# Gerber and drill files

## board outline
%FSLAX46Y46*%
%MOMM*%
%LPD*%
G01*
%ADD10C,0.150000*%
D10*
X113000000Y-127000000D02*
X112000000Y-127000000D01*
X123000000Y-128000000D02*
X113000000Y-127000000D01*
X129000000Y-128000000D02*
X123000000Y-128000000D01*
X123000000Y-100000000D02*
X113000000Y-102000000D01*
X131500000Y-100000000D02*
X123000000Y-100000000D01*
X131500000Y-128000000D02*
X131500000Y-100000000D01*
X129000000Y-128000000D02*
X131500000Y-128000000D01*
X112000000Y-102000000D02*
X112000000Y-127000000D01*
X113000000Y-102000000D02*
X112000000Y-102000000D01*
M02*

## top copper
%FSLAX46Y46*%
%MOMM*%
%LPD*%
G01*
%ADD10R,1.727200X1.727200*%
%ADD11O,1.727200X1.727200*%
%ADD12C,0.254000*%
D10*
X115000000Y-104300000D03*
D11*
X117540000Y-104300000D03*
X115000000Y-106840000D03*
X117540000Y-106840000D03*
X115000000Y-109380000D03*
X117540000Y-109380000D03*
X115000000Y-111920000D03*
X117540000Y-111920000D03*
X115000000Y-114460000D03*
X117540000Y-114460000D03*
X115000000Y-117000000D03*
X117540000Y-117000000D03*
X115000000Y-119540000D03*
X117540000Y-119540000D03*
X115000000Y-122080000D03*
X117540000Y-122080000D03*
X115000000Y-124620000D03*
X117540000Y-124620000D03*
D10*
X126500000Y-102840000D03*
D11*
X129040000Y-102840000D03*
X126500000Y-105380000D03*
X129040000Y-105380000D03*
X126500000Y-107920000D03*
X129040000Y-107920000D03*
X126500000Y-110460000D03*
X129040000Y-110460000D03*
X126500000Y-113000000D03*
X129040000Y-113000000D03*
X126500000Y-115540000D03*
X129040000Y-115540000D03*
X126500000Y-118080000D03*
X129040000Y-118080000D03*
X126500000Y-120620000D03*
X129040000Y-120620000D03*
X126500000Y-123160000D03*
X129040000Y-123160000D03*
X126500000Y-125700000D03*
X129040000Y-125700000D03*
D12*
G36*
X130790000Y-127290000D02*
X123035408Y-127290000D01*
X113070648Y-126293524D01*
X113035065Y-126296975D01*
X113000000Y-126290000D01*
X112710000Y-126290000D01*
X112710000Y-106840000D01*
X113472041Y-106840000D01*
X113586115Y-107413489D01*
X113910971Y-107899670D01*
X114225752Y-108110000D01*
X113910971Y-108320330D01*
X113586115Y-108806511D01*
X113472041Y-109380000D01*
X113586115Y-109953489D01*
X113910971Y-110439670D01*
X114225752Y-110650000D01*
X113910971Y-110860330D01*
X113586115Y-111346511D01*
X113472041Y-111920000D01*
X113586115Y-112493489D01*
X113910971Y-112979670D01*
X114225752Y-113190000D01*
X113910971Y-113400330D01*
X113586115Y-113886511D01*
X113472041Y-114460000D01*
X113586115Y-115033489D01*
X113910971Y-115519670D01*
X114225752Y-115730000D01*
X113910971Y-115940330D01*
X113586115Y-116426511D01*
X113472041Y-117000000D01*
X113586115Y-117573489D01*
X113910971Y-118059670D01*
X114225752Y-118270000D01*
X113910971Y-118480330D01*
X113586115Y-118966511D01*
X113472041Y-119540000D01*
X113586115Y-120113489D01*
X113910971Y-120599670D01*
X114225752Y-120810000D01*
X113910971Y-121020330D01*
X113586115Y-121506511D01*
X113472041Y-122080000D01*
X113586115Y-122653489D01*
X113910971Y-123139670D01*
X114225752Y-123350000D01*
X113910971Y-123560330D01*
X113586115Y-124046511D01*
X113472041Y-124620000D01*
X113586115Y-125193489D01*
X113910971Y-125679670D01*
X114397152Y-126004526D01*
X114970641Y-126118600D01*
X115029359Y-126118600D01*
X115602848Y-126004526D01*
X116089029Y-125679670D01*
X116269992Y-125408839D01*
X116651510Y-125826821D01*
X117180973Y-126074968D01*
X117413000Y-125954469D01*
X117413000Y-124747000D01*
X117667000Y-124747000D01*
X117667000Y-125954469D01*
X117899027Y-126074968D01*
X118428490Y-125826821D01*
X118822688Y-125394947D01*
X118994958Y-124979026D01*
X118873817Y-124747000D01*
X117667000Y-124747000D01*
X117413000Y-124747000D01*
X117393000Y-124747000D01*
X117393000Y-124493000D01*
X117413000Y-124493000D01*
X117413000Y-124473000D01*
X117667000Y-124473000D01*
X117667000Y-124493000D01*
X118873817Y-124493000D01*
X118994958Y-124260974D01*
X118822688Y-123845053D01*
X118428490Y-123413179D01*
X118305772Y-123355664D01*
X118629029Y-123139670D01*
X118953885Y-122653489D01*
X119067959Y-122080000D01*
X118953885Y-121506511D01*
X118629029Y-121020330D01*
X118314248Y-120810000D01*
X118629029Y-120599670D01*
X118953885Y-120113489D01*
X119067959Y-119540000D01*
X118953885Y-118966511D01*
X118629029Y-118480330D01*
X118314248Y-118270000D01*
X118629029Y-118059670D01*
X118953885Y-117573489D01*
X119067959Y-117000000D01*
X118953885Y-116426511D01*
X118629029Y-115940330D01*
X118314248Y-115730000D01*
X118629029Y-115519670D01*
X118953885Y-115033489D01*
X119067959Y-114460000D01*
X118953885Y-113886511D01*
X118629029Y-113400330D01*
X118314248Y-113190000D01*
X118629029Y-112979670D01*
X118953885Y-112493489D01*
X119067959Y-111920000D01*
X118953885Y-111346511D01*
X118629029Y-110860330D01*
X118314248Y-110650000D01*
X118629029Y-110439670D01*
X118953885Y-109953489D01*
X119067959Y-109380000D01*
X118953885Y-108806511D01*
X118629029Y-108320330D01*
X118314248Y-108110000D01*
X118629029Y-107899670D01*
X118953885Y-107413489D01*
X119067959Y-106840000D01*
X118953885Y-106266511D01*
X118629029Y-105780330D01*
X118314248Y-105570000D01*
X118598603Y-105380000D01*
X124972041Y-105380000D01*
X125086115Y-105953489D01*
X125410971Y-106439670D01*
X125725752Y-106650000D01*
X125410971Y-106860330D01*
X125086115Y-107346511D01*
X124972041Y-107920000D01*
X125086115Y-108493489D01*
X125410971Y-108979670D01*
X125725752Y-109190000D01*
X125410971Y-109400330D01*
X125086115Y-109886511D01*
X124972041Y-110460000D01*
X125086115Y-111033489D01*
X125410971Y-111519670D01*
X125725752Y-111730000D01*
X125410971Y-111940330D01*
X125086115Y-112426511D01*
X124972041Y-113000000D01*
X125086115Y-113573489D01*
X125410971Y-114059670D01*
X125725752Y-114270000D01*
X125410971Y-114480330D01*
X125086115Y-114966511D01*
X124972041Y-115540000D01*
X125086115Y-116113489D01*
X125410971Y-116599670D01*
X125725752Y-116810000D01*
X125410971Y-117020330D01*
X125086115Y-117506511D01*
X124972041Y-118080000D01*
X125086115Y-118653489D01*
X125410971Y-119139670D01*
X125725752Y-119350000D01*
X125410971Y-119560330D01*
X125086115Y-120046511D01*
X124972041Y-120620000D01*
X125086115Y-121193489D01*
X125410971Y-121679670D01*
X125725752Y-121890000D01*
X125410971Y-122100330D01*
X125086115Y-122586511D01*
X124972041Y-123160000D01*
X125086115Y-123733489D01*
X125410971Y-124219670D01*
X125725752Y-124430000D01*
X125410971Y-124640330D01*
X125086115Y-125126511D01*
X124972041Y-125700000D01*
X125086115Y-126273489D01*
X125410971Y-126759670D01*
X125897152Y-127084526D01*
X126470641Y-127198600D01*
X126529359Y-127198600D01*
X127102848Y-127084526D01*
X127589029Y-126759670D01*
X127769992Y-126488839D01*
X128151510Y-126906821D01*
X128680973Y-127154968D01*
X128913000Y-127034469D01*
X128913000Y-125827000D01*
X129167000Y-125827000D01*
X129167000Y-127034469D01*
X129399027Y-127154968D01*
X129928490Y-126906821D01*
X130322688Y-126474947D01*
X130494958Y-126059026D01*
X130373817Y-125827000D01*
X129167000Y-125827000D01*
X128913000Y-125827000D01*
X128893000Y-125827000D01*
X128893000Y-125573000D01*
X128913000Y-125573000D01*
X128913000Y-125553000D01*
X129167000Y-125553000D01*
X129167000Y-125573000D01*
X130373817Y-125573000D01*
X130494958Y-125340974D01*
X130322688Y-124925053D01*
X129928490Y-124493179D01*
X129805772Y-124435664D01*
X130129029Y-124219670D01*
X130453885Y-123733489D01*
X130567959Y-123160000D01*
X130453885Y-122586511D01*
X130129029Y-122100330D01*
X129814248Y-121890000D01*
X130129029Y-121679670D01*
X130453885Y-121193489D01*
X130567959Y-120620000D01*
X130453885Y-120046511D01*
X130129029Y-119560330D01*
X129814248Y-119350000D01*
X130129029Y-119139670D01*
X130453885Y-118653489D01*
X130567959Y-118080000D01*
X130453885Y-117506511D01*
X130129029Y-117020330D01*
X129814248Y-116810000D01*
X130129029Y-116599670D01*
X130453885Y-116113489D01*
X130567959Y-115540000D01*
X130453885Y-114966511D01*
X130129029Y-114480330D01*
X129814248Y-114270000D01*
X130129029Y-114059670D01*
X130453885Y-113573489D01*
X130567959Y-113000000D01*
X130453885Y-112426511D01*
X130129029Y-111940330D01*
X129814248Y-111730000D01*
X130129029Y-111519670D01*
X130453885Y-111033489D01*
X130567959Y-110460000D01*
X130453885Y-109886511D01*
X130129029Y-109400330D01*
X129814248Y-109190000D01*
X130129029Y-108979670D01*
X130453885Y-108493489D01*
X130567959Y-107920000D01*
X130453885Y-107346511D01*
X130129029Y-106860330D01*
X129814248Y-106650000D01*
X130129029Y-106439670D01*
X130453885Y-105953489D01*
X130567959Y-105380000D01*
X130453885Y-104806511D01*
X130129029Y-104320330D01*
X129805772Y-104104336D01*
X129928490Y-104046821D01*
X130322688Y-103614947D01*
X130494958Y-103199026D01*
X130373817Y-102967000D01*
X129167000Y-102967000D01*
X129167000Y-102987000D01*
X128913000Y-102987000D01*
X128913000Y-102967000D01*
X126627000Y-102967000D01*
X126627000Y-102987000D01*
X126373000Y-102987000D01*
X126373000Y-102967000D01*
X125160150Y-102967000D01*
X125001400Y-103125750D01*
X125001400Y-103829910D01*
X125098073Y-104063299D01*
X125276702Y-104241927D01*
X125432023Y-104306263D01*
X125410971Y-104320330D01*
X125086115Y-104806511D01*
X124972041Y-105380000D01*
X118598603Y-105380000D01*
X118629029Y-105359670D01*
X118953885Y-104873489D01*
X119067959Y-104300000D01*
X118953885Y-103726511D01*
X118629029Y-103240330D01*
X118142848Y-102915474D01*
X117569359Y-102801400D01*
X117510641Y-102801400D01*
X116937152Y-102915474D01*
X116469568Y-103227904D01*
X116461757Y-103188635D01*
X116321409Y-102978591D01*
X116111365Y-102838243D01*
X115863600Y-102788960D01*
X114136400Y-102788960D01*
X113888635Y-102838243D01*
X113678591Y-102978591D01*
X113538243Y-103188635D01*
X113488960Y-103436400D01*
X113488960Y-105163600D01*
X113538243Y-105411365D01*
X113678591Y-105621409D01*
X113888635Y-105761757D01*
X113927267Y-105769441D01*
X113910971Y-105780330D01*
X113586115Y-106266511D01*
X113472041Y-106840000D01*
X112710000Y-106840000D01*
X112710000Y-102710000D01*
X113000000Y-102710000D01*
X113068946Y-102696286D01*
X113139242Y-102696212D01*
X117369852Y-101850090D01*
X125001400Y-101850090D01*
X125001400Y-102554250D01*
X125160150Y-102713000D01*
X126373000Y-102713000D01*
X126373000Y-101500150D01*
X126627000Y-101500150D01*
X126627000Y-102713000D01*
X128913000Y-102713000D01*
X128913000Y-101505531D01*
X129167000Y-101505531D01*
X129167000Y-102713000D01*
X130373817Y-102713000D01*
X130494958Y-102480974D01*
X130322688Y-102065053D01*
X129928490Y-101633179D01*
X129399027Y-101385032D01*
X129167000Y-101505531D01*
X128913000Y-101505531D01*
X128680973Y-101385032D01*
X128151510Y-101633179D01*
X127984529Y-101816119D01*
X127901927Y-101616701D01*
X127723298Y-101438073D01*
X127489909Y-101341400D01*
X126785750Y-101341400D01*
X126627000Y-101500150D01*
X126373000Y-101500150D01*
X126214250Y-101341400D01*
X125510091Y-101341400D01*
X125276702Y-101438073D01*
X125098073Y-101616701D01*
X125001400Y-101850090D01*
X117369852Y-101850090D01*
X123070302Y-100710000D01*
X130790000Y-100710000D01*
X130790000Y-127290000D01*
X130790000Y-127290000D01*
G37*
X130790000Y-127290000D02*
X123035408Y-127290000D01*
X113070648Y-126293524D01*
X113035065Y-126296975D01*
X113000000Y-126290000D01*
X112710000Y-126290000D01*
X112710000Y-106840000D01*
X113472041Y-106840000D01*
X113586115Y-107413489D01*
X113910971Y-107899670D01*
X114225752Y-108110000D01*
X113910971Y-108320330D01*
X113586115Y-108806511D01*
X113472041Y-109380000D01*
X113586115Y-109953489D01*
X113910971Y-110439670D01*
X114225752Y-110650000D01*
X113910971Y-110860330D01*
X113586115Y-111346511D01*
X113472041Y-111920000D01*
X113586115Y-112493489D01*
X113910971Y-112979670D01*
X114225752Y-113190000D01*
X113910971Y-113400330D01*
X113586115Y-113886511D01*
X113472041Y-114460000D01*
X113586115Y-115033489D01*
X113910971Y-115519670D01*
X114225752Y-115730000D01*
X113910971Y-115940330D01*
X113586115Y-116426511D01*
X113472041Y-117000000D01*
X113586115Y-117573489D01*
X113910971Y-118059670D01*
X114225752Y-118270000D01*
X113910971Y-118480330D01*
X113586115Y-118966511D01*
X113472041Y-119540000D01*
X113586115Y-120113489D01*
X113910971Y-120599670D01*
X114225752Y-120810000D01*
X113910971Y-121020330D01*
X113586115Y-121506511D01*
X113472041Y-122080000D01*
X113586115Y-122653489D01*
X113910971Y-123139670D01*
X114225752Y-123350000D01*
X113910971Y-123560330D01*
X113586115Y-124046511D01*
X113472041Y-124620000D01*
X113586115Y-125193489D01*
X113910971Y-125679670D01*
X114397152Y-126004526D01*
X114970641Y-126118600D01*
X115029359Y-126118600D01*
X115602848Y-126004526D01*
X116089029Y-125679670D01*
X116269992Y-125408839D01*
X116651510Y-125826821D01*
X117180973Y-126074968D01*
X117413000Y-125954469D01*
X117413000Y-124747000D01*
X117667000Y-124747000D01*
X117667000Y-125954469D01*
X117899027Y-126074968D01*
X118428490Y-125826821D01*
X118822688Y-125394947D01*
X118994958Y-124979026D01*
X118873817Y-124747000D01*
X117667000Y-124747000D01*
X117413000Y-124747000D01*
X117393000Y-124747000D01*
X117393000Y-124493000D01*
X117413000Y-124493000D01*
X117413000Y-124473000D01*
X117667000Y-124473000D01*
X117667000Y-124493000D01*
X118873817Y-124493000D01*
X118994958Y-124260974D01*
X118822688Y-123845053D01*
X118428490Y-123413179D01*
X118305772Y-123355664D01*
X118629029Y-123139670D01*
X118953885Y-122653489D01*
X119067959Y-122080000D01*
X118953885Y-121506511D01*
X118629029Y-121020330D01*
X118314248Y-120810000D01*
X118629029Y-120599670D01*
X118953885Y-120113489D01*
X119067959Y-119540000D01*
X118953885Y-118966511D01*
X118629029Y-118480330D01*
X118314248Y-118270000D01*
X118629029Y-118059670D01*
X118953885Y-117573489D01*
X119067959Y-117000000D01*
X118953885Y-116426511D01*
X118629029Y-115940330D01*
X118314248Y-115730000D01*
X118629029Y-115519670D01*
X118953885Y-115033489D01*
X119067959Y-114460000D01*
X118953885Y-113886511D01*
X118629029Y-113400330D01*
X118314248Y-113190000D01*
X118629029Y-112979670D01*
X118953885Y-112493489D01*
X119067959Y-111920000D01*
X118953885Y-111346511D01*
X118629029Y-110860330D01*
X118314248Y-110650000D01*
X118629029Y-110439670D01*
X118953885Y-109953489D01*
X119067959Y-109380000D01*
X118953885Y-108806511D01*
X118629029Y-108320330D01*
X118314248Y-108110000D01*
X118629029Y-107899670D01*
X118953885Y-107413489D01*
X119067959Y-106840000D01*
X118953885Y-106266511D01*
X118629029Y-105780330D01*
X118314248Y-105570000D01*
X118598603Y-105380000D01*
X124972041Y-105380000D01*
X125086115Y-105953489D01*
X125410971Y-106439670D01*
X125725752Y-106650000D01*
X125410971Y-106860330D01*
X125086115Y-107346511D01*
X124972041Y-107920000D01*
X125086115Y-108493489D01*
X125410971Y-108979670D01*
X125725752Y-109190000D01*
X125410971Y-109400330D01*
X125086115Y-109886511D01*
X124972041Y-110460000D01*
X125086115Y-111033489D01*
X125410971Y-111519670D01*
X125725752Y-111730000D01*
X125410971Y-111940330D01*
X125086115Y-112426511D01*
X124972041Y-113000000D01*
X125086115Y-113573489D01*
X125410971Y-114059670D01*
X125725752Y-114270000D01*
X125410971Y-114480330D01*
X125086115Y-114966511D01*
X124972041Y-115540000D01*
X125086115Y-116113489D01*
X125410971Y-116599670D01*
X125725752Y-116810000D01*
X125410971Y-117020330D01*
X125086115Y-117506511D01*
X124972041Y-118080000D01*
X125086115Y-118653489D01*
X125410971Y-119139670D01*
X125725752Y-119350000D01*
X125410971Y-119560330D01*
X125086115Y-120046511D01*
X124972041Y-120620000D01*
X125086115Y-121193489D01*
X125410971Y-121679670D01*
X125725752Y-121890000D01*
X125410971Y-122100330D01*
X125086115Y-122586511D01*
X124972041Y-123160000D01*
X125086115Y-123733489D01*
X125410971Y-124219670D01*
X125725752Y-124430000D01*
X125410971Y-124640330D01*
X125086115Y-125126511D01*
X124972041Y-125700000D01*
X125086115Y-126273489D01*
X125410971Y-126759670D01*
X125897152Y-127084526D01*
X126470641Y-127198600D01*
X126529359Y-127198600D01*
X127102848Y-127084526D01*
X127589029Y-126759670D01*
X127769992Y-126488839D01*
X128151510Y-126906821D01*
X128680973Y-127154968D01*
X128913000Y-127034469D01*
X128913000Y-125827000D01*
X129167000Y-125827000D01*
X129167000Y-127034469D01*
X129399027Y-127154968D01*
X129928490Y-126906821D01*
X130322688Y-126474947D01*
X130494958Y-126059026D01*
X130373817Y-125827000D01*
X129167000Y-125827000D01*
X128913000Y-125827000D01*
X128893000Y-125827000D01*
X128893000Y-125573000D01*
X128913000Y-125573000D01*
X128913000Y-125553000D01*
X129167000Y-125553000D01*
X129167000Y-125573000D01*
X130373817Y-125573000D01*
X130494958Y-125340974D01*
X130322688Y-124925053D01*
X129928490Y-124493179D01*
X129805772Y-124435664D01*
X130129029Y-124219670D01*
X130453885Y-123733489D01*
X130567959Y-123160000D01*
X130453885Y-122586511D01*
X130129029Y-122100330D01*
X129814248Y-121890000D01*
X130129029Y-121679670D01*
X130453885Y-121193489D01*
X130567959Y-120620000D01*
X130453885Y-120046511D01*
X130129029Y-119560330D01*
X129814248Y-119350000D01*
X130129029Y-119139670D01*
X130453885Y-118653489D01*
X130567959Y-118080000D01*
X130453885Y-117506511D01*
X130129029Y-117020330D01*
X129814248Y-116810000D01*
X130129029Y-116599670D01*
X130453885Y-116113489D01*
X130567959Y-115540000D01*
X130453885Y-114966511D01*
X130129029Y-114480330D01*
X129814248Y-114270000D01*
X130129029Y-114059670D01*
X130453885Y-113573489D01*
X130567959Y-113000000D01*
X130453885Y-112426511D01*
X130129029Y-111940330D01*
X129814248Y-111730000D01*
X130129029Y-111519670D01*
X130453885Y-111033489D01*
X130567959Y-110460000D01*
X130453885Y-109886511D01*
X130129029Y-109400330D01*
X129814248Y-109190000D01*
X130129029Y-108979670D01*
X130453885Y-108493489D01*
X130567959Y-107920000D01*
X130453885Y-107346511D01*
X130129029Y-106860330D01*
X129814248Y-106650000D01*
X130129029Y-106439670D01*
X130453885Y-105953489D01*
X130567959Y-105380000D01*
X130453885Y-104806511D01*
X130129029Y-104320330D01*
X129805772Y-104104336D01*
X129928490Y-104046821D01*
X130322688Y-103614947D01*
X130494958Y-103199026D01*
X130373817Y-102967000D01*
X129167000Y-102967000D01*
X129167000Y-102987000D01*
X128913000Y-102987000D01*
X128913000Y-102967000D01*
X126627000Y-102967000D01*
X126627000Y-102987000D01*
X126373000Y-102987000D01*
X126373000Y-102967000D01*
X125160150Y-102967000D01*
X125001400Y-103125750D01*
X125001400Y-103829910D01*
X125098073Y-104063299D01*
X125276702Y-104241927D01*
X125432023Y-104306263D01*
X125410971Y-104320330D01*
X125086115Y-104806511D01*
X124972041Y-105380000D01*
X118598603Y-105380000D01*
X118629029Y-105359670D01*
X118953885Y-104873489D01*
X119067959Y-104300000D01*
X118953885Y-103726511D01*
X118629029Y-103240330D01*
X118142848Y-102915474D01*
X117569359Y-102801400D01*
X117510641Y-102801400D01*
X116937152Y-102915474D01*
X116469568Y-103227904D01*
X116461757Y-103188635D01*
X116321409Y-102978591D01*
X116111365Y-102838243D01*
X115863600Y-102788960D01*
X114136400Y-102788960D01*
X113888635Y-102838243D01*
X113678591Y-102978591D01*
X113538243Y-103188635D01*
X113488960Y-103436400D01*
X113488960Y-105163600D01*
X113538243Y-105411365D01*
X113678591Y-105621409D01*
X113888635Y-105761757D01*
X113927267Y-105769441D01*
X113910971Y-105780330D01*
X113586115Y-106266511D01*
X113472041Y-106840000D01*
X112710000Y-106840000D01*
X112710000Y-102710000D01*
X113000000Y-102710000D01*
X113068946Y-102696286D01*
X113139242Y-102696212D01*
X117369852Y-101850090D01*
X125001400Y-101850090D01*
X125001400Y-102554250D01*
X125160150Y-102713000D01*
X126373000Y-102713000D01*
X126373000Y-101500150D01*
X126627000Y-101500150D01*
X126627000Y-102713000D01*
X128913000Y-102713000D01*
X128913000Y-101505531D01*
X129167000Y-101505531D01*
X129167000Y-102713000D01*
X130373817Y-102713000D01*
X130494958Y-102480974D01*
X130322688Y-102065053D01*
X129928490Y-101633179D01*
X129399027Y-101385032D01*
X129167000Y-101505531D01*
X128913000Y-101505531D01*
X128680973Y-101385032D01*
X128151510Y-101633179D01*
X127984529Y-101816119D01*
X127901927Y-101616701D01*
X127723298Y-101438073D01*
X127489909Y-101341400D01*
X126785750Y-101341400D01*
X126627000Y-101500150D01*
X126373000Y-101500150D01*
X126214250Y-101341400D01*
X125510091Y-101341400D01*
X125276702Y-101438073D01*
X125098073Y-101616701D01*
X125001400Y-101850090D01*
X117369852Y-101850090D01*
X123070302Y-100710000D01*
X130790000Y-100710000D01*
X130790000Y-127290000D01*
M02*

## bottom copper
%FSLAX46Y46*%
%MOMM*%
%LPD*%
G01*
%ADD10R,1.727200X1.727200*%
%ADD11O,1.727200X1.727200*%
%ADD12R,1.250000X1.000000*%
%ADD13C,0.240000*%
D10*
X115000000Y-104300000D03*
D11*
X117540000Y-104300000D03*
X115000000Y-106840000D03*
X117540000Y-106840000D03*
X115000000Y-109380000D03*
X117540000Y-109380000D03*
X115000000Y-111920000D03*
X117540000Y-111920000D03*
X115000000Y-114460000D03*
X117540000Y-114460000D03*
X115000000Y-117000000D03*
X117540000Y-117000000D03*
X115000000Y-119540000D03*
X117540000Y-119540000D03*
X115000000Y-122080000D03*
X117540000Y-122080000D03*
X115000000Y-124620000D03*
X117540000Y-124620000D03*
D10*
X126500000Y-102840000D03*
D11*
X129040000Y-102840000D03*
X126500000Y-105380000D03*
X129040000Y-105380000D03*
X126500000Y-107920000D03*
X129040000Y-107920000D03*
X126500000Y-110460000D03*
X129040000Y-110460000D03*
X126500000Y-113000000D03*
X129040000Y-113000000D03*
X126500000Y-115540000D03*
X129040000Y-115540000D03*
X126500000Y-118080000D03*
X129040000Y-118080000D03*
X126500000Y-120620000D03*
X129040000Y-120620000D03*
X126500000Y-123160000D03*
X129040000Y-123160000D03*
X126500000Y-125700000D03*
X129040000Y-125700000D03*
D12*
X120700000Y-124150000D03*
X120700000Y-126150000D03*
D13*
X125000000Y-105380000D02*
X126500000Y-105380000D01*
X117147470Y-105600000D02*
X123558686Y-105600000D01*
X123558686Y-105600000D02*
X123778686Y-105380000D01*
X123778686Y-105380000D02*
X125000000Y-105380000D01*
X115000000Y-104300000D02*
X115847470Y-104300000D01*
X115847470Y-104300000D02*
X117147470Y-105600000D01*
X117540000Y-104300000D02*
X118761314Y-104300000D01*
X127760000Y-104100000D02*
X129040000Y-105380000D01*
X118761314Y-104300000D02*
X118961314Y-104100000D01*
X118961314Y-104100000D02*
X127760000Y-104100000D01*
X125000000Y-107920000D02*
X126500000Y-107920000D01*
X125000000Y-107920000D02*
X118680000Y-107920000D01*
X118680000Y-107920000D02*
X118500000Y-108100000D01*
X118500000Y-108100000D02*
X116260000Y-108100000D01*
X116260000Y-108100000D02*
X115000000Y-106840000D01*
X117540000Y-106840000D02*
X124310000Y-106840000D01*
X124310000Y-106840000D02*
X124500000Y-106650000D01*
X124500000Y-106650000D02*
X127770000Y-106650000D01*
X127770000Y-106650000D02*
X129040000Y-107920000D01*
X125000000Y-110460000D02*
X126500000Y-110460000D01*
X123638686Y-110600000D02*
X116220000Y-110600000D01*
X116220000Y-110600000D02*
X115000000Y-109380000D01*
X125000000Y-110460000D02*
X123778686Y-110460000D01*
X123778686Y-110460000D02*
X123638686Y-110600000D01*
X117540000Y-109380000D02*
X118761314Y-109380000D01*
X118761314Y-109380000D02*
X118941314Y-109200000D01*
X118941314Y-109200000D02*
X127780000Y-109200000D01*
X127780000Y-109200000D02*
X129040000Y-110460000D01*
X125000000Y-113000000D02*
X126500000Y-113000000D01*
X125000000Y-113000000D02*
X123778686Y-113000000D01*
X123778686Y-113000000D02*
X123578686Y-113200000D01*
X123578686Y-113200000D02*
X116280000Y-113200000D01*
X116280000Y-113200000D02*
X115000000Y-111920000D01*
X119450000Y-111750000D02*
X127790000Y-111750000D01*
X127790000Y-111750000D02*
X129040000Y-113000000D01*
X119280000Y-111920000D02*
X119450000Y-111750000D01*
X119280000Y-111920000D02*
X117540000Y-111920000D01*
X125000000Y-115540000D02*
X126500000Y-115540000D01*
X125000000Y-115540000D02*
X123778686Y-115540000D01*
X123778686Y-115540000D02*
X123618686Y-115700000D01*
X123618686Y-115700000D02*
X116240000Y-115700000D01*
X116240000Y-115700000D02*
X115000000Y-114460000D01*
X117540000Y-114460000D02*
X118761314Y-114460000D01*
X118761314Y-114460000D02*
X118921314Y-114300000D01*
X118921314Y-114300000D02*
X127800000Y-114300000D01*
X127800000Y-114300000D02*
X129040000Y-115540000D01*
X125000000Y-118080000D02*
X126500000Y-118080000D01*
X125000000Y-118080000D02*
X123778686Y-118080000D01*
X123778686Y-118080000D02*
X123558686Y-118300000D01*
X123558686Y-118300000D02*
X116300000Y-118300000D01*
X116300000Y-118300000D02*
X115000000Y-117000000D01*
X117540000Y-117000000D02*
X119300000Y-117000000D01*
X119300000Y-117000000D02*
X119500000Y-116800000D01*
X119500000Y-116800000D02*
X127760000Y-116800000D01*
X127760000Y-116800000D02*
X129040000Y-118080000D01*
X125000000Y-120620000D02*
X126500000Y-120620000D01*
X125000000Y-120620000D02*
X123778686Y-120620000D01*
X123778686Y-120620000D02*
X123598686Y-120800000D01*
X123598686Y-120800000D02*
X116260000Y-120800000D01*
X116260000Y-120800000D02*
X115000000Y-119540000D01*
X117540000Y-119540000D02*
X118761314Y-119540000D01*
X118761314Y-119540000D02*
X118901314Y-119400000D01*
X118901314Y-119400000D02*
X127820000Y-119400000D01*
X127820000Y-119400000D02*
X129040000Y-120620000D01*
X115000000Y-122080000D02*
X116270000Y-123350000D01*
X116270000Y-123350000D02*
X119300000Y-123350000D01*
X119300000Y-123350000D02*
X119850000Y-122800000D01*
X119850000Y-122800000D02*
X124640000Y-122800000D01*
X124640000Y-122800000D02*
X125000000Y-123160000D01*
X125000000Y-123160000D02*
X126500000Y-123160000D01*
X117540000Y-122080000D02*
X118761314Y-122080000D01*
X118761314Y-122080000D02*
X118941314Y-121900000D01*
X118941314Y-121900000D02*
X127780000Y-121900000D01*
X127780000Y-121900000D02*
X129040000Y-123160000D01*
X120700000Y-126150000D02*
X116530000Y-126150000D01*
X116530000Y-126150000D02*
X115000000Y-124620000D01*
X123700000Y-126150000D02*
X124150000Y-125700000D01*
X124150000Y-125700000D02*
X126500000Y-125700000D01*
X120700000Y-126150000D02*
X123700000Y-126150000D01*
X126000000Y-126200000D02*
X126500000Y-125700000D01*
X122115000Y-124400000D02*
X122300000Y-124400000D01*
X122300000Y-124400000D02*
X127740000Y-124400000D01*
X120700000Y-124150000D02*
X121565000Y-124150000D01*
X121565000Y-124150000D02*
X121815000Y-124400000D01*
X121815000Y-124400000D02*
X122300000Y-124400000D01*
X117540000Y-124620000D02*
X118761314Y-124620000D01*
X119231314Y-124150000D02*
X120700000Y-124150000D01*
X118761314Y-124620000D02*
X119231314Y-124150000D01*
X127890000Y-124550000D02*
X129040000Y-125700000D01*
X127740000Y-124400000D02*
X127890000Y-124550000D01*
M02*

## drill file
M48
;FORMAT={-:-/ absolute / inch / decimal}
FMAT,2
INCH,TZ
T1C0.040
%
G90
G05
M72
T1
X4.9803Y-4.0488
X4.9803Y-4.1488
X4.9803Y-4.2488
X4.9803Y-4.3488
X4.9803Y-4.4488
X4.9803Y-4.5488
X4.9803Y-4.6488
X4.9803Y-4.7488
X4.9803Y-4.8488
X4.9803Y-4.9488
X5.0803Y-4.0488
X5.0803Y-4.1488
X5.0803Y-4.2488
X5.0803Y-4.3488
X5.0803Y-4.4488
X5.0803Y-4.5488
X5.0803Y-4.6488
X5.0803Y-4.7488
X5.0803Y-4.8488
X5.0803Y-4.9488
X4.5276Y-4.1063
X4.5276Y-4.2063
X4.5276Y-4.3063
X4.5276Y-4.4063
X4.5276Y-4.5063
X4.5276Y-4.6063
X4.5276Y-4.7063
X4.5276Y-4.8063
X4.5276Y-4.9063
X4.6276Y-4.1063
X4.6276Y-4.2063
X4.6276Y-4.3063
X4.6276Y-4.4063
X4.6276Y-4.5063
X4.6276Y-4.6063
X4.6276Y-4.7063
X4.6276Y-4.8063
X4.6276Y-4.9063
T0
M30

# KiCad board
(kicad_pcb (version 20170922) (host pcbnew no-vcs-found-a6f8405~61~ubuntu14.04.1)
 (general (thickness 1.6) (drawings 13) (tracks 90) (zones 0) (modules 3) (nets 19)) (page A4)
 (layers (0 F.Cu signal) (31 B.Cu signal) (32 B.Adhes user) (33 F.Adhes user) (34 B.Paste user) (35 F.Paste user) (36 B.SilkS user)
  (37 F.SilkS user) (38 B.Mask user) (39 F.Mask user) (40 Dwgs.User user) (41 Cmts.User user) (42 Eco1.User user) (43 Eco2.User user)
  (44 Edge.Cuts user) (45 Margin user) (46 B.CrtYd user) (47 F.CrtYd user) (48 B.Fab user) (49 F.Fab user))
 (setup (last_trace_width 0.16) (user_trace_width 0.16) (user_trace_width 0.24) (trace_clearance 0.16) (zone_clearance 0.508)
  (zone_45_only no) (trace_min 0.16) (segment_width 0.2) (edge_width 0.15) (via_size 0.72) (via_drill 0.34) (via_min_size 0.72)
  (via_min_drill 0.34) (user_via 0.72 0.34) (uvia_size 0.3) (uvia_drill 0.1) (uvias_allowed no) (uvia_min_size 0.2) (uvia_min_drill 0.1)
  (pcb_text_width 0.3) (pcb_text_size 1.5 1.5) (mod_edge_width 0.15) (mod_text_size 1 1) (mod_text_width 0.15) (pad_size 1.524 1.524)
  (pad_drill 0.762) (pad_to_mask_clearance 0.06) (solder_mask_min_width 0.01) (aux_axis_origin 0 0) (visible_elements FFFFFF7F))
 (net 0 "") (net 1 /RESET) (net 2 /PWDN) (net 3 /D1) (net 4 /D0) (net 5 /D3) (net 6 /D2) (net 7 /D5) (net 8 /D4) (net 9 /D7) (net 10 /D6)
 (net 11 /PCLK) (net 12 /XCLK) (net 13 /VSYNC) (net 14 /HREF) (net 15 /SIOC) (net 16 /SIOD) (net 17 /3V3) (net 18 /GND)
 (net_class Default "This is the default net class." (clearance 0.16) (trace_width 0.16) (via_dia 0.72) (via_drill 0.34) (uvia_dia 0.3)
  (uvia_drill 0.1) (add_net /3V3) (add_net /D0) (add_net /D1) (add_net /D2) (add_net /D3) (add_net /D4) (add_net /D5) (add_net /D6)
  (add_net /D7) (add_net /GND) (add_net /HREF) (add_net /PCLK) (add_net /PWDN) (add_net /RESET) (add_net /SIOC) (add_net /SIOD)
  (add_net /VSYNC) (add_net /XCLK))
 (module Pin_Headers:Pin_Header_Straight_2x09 (layer F.Cu) (at 115 104.3)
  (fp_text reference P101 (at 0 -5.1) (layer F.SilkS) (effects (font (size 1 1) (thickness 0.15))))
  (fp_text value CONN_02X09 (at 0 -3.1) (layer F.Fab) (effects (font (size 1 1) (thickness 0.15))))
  (pad 1 thru_hole rect (at 0 0) (size 1.7272 1.7272) (drill 1.016) (layers *.Cu *.Mask F.SilkS) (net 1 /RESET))
  (pad 2 thru_hole oval (at 2.54 0) (size 1.7272 1.7272) (drill 1.016) (layers *.Cu *.Mask F.SilkS) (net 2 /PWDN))
  (pad 3 thru_hole oval (at 0 2.54) (size 1.7272 1.7272) (drill 1.016) (layers *.Cu *.Mask F.SilkS) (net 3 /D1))
  (pad 4 thru_hole oval (at 2.54 2.54) (size 1.7272 1.7272) (drill 1.016) (layers *.Cu *.Mask F.SilkS) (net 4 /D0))
  (pad 5 thru_hole oval (at 0 5.08) (size 1.7272 1.7272) (drill 1.016) (layers *.Cu *.Mask F.SilkS) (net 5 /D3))
  (pad 6 thru_hole oval (at 2.54 5.08) (size 1.7272 1.7272) (drill 1.016) (layers *.Cu *.Mask F.SilkS) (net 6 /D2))
  (pad 7 thru_hole oval (at 0 7.62) (size 1.7272 1.7272) (drill 1.016) (layers *.Cu *.Mask F.SilkS) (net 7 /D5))
  (pad 8 thru_hole oval (at 2.54 7.62) (size 1.7272 1.7272) (drill 1.016) (layers *.Cu *.Mask F.SilkS) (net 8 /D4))
  (pad 9 thru_hole oval (at 0 10.16) (size 1.7272 1.7272) (drill 1.016) (layers *.Cu *.Mask F.SilkS) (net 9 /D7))
  (pad 10 thru_hole oval (at 2.54 10.16) (size 1.7272 1.7272) (drill 1.016) (layers *.Cu *.Mask F.SilkS) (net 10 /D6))
  (pad 11 thru_hole oval (at 0 12.7) (size 1.7272 1.7272) (drill 1.016) (layers *.Cu *.Mask F.SilkS) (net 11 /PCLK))
  (pad 12 thru_hole oval (at 2.54 12.7) (size 1.7272 1.7272) (drill 1.016) (layers *.Cu *.Mask F.SilkS) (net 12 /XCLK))
  (pad 13 thru_hole oval (at 0 15.24) (size 1.7272 1.7272) (drill 1.016) (layers *.Cu *.Mask F.SilkS) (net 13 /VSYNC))
  (pad 14 thru_hole oval (at 2.54 15.24) (size 1.7272 1.7272) (drill 1.016) (layers *.Cu *.Mask F.SilkS) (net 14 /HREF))
  (pad 15 thru_hole oval (at 0 17.78) (size 1.7272 1.7272) (drill 1.016) (layers *.Cu *.Mask F.SilkS) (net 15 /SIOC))
  (pad 16 thru_hole oval (at 2.54 17.78) (size 1.7272 1.7272) (drill 1.016) (layers *.Cu *.Mask F.SilkS) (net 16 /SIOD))
  (pad 17 thru_hole oval (at 0 20.32) (size 1.7272 1.7272) (drill 1.016) (layers *.Cu *.Mask F.SilkS) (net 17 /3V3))
  (pad 18 thru_hole oval (at 2.54 20.32) (size 1.7272 1.7272) (drill 1.016) (layers *.Cu *.Mask F.SilkS) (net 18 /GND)))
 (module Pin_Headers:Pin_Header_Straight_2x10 (layer F.Cu) (at 126.5 102.84)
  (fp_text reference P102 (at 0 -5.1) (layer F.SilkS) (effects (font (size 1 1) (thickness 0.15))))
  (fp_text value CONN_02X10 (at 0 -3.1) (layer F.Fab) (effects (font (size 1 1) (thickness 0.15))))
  (pad 1 thru_hole rect (at 0 0) (size 1.7272 1.7272) (drill 1.016) (layers *.Cu *.Mask F.SilkS) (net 18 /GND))
  (pad 2 thru_hole oval (at 2.54 0) (size 1.7272 1.7272) (drill 1.016) (layers *.Cu *.Mask F.SilkS) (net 18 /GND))
  (pad 3 thru_hole oval (at 0 2.54) (size 1.7272 1.7272) (drill 1.016) (layers *.Cu *.Mask F.SilkS) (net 1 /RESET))
  (pad 4 thru_hole oval (at 2.54 2.54) (size 1.7272 1.7272) (drill 1.016) (layers *.Cu *.Mask F.SilkS) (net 2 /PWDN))
  (pad 5 thru_hole oval (at 0 5.08) (size 1.7272 1.7272) (drill 1.016) (layers *.Cu *.Mask F.SilkS) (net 3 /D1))
  (pad 6 thru_hole oval (at 2.54 5.08) (size 1.7272 1.7272) (drill 1.016) (layers *.Cu *.Mask F.SilkS) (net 4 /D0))
  (pad 7 thru_hole oval (at 0 7.62) (size 1.7272 1.7272) (drill 1.016) (layers *.Cu *.Mask F.SilkS) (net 5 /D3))
  (pad 8 thru_hole oval (at 2.54 7.62) (size 1.7272 1.7272) (drill 1.016) (layers *.Cu *.Mask F.SilkS) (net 6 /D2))
  (pad 9 thru_hole oval (at 0 10.16) (size 1.7272 1.7272) (drill 1.016) (layers *.Cu *.Mask F.SilkS) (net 7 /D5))
  (pad 10 thru_hole oval (at 2.54 10.16) (size 1.7272 1.7272) (drill 1.016) (layers *.Cu *.Mask F.SilkS) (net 8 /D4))
  (pad 11 thru_hole oval (at 0 12.7) (size 1.7272 1.7272) (drill 1.016) (layers *.Cu *.Mask F.SilkS) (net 9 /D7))
  (pad 12 thru_hole oval (at 2.54 12.7) (size 1.7272 1.7272) (drill 1.016) (layers *.Cu *.Mask F.SilkS) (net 10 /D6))
  (pad 13 thru_hole oval (at 0 15.24) (size 1.7272 1.7272) (drill 1.016) (layers *.Cu *.Mask F.SilkS) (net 11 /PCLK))
  (pad 14 thru_hole oval (at 2.54 15.24) (size 1.7272 1.7272) (drill 1.016) (layers *.Cu *.Mask F.SilkS) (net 12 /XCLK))
  (pad 15 thru_hole oval (at 0 17.78) (size 1.7272 1.7272) (drill 1.016) (layers *.Cu *.Mask F.SilkS) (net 13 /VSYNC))
  (pad 16 thru_hole oval (at 2.54 17.78) (size 1.7272 1.7272) (drill 1.016) (layers *.Cu *.Mask F.SilkS) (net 14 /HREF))
  (pad 17 thru_hole oval (at 0 20.32) (size 1.7272 1.7272) (drill 1.016) (layers *.Cu *.Mask F.SilkS) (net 15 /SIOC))
  (pad 18 thru_hole oval (at 2.54 20.32) (size 1.7272 1.7272) (drill 1.016) (layers *.Cu *.Mask F.SilkS) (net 16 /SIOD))
  (pad 19 thru_hole oval (at 0 22.86) (size 1.7272 1.7272) (drill 1.016) (layers *.Cu *.Mask F.SilkS) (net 17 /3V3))
  (pad 20 thru_hole oval (at 2.54 22.86) (size 1.7272 1.7272) (drill 1.016) (layers *.Cu *.Mask F.SilkS) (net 18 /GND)))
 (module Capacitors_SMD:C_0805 (layer B.Cu) (at 120.7 125.15 90)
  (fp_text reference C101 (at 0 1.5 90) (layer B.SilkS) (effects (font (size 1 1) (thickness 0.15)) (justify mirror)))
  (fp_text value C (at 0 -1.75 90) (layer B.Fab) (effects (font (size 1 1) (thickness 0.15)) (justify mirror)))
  (pad 2 smd rect (at 1 0 90) (size 1 1.25) (layers B.Cu B.Paste B.Mask) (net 18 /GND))
  (pad 1 smd rect (at -1 0 90) (size 1 1.25) (layers B.Cu B.Paste B.Mask) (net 17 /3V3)))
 (gr_line (start 113 127) (end 112 127) (layer Edge.Cuts) (width 0.15))
 (gr_line (start 123 128) (end 113 127) (layer Edge.Cuts) (width 0.15))
 (gr_line (start 129 128) (end 123 128) (layer Edge.Cuts) (width 0.15))
 (gr_line (start 123 100) (end 113 102) (layer Edge.Cuts) (width 0.15))
 (gr_line (start 131.5 100) (end 123 100) (layer Edge.Cuts) (width 0.15))
 (gr_line (start 131.5 128) (end 131.5 100) (layer Edge.Cuts) (width 0.15))
 (gr_line (start 129 128) (end 131.5 128) (layer Edge.Cuts) (width 0.15))
 (gr_line (start 112 102) (end 112 127) (layer Edge.Cuts) (width 0.15))
 (gr_line (start 113 102) (end 112 102) (layer Edge.Cuts) (width 0.15))
 (segment (start 125 105.38) (end 126.5 105.38) (width 0.24) (layer B.Cu) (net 1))
 (segment (start 117.14747 105.6) (end 123.558686 105.6) (width 0.24) (layer B.Cu) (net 1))
 (segment (start 123.558686 105.6) (end 123.778686 105.38) (width 0.24) (layer B.Cu) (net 1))
 (segment (start 123.778686 105.38) (end 125 105.38) (width 0.24) (layer B.Cu) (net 1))
 (segment (start 115 104.3) (end 115.84747 104.3) (width 0.24) (layer B.Cu) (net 1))
 (segment (start 115.84747 104.3) (end 117.14747 105.6) (width 0.24) (layer B.Cu) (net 1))
 (segment (start 117.54 104.3) (end 118.761314 104.3) (width 0.24) (layer B.Cu) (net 2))
 (segment (start 127.76 104.1) (end 129.04 105.38) (width 0.24) (layer B.Cu) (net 2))
 (segment (start 118.761314 104.3) (end 118.961314 104.1) (width 0.24) (layer B.Cu) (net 2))
 (segment (start 118.961314 104.1) (end 127.76 104.1) (width 0.24) (layer B.Cu) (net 2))
 (segment (start 125 107.92) (end 126.5 107.92) (width 0.24) (layer B.Cu) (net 3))
 (segment (start 125 107.92) (end 118.68 107.92) (width 0.24) (layer B.Cu) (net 3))
 (segment (start 118.68 107.92) (end 118.5 108.1) (width 0.24) (layer B.Cu) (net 3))
 (segment (start 118.5 108.1) (end 116.26 108.1) (width 0.24) (layer B.Cu) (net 3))
 (segment (start 116.26 108.1) (end 115 106.84) (width 0.24) (layer B.Cu) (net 3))
 (segment (start 117.54 106.84) (end 124.31 106.84) (width 0.24) (layer B.Cu) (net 4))
 (segment (start 124.31 106.84) (end 124.5 106.65) (width 0.24) (layer B.Cu) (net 4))
 (segment (start 124.5 106.65) (end 127.77 106.65) (width 0.24) (layer B.Cu) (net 4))
 (segment (start 127.77 106.65) (end 129.04 107.92) (width 0.24) (layer B.Cu) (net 4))
 (segment (start 125 110.46) (end 126.5 110.46) (width 0.24) (layer B.Cu) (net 5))
 (segment (start 123.638686 110.6) (end 116.22 110.6) (width 0.24) (layer B.Cu) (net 5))
 (segment (start 116.22 110.6) (end 115 109.38) (width 0.24) (layer B.Cu) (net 5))
 (segment (start 125 110.46) (end 123.778686 110.46) (width 0.24) (layer B.Cu) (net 5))
 (segment (start 123.778686 110.46) (end 123.638686 110.6) (width 0.24) (layer B.Cu) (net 5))
 (segment (start 117.54 109.38) (end 118.761314 109.38) (width 0.24) (layer B.Cu) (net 6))
 (segment (start 118.761314 109.38) (end 118.941314 109.2) (width 0.24) (layer B.Cu) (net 6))
 (segment (start 118.941314 109.2) (end 127.78 109.2) (width 0.24) (layer B.Cu) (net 6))
 (segment (start 127.78 109.2) (end 129.04 110.46) (width 0.24) (layer B.Cu) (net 6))
 (segment (start 125 113) (end 126.5 113) (width 0.24) (layer B.Cu) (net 7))
 (segment (start 125 113) (end 123.778686 113) (width 0.24) (layer B.Cu) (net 7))
 (segment (start 123.778686 113) (end 123.578686 113.2) (width 0.24) (layer B.Cu) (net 7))
 (segment (start 123.578686 113.2) (end 116.28 113.2) (width 0.24) (layer B.Cu) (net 7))
 (segment (start 116.28 113.2) (end 115 111.92) (width 0.24) (layer B.Cu) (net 7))
 (segment (start 119.45 111.75) (end 127.79 111.75) (width 0.24) (layer B.Cu) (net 8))
 (segment (start 127.79 111.75) (end 129.04 113) (width 0.24) (layer B.Cu) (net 8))
 (segment (start 119.28 111.92) (end 119.45 111.75) (width 0.24) (layer B.Cu) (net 8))
 (segment (start 119.28 111.92) (end 117.54 111.92) (width 0.24) (layer B.Cu) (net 8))
 (segment (start 125 115.54) (end 126.5 115.54) (width 0.24) (layer B.Cu) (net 9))
 (segment (start 125 115.54) (end 123.778686 115.54) (width 0.24) (layer B.Cu) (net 9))
 (segment (start 123.778686 115.54) (end 123.618686 115.7) (width 0.24) (layer B.Cu) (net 9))
 (segment (start 123.618686 115.7) (end 116.24 115.7) (width 0.24) (layer B.Cu) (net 9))
 (segment (start 116.24 115.7) (end 115 114.46) (width 0.24) (layer B.Cu) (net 9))
 (segment (start 117.54 114.46) (end 118.761314 114.46) (width 0.24) (layer B.Cu) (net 10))
 (segment (start 118.761314 114.46) (end 118.921314 114.3) (width 0.24) (layer B.Cu) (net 10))
 (segment (start 118.921314 114.3) (end 127.8 114.3) (width 0.24) (layer B.Cu) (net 10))
 (segment (start 127.8 114.3) (end 129.04 115.54) (width 0.24) (layer B.Cu) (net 10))
 (segment (start 125 118.08) (end 126.5 118.08) (width 0.24) (layer B.Cu) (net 11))
 (segment (start 125 118.08) (end 123.778686 118.08) (width 0.24) (layer B.Cu) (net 11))
 (segment (start 123.778686 118.08) (end 123.558686 118.3) (width 0.24) (layer B.Cu) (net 11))
 (segment (start 123.558686 118.3) (end 116.3 118.3) (width 0.24) (layer B.Cu) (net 11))
 (segment (start 116.3 118.3) (end 115 117) (width 0.24) (layer B.Cu) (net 11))
 (segment (start 117.54 117) (end 119.3 117) (width 0.24) (layer B.Cu) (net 12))
 (segment (start 119.3 117) (end 119.5 116.8) (width 0.24) (layer B.Cu) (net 12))
 (segment (start 119.5 116.8) (end 127.76 116.8) (width 0.24) (layer B.Cu) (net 12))
 (segment (start 127.76 116.8) (end 129.04 118.08) (width 0.24) (layer B.Cu) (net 12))
 (segment (start 125 120.62) (end 126.5 120.62) (width 0.24) (layer B.Cu) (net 13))
 (segment (start 125 120.62) (end 123.778686 120.62) (width 0.24) (layer B.Cu) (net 13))
 (segment (start 123.778686 120.62) (end 123.598686 120.8) (width 0.24) (layer B.Cu) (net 13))
 (segment (start 123.598686 120.8) (end 116.26 120.8) (width 0.24) (layer B.Cu) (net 13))
 (segment (start 116.26 120.8) (end 115 119.54) (width 0.24) (layer B.Cu) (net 13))
 (segment (start 117.54 119.54) (end 118.761314 119.54) (width 0.24) (layer B.Cu) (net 14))
 (segment (start 118.761314 119.54) (end 118.901314 119.4) (width 0.24) (layer B.Cu) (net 14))
 (segment (start 118.901314 119.4) (end 127.82 119.4) (width 0.24) (layer B.Cu) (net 14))
 (segment (start 127.82 119.4) (end 129.04 120.62) (width 0.24) (layer B.Cu) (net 14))
 (segment (start 115 122.08) (end 116.27 123.35) (width 0.24) (layer B.Cu) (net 15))
 (segment (start 116.27 123.35) (end 119.3 123.35) (width 0.24) (layer B.Cu) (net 15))
 (segment (start 119.3 123.35) (end 119.85 122.8) (width 0.24) (layer B.Cu) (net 15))
 (segment (start 119.85 122.8) (end 124.64 122.8) (width 0.24) (layer B.Cu) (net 15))
 (segment (start 124.64 122.8) (end 125 123.16) (width 0.24) (layer B.Cu) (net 15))
 (segment (start 125 123.16) (end 126.5 123.16) (width 0.24) (layer B.Cu) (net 15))
 (segment (start 117.54 122.08) (end 118.761314 122.08) (width 0.24) (layer B.Cu) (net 16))
 (segment (start 118.761314 122.08) (end 118.941314 121.9) (width 0.24) (layer B.Cu) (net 16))
 (segment (start 118.941314 121.9) (end 127.78 121.9) (width 0.24) (layer B.Cu) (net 16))
 (segment (start 127.78 121.9) (end 129.04 123.16) (width 0.24) (layer B.Cu) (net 16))
 (segment (start 120.7 126.15) (end 116.53 126.15) (width 0.24) (layer B.Cu) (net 17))
 (segment (start 116.53 126.15) (end 115 124.62) (width 0.24) (layer B.Cu) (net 17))
 (segment (start 123.7 126.15) (end 124.15 125.7) (width 0.24) (layer B.Cu) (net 17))
 (segment (start 124.15 125.7) (end 126.5 125.7) (width 0.24) (layer B.Cu) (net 17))
 (segment (start 120.7 126.15) (end 123.7 126.15) (width 0.24) (layer B.Cu) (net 17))
 (segment (start 126 126.2) (end 126.5 125.7) (width 0.24) (layer B.Cu) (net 17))
 (segment (start 122.115 124.4) (end 122.3 124.4) (width 0.24) (layer B.Cu) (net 18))
 (segment (start 122.3 124.4) (end 127.74 124.4) (width 0.24) (layer B.Cu) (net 18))
 (segment (start 120.7 124.15) (end 121.565 124.15) (width 0.24) (layer B.Cu) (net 18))
 (segment (start 121.565 124.15) (end 121.815 124.4) (width 0.24) (layer B.Cu) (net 18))
 (segment (start 121.815 124.4) (end 122.3 124.4) (width 0.24) (layer B.Cu) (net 18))
 (segment (start 117.54 124.62) (end 118.761314 124.62) (width 0.24) (layer B.Cu) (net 18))
 (segment (start 119.231314 124.15) (end 120.7 124.15) (width 0.24) (layer B.Cu) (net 18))
 (segment (start 118.761314 124.62) (end 119.231314 124.15) (width 0.24) (layer B.Cu) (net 18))
 (segment (start 127.89 124.55) (end 129.04 125.7) (width 0.24) (layer B.Cu) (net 18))
 (segment (start 127.74 124.4) (end 127.89 124.55) (width 0.24) (layer B.Cu) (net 18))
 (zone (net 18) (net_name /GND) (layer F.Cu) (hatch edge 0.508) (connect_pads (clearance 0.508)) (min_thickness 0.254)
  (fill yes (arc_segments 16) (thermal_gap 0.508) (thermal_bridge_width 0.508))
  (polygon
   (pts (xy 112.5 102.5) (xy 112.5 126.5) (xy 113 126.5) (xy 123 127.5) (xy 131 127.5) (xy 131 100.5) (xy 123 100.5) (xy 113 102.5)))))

